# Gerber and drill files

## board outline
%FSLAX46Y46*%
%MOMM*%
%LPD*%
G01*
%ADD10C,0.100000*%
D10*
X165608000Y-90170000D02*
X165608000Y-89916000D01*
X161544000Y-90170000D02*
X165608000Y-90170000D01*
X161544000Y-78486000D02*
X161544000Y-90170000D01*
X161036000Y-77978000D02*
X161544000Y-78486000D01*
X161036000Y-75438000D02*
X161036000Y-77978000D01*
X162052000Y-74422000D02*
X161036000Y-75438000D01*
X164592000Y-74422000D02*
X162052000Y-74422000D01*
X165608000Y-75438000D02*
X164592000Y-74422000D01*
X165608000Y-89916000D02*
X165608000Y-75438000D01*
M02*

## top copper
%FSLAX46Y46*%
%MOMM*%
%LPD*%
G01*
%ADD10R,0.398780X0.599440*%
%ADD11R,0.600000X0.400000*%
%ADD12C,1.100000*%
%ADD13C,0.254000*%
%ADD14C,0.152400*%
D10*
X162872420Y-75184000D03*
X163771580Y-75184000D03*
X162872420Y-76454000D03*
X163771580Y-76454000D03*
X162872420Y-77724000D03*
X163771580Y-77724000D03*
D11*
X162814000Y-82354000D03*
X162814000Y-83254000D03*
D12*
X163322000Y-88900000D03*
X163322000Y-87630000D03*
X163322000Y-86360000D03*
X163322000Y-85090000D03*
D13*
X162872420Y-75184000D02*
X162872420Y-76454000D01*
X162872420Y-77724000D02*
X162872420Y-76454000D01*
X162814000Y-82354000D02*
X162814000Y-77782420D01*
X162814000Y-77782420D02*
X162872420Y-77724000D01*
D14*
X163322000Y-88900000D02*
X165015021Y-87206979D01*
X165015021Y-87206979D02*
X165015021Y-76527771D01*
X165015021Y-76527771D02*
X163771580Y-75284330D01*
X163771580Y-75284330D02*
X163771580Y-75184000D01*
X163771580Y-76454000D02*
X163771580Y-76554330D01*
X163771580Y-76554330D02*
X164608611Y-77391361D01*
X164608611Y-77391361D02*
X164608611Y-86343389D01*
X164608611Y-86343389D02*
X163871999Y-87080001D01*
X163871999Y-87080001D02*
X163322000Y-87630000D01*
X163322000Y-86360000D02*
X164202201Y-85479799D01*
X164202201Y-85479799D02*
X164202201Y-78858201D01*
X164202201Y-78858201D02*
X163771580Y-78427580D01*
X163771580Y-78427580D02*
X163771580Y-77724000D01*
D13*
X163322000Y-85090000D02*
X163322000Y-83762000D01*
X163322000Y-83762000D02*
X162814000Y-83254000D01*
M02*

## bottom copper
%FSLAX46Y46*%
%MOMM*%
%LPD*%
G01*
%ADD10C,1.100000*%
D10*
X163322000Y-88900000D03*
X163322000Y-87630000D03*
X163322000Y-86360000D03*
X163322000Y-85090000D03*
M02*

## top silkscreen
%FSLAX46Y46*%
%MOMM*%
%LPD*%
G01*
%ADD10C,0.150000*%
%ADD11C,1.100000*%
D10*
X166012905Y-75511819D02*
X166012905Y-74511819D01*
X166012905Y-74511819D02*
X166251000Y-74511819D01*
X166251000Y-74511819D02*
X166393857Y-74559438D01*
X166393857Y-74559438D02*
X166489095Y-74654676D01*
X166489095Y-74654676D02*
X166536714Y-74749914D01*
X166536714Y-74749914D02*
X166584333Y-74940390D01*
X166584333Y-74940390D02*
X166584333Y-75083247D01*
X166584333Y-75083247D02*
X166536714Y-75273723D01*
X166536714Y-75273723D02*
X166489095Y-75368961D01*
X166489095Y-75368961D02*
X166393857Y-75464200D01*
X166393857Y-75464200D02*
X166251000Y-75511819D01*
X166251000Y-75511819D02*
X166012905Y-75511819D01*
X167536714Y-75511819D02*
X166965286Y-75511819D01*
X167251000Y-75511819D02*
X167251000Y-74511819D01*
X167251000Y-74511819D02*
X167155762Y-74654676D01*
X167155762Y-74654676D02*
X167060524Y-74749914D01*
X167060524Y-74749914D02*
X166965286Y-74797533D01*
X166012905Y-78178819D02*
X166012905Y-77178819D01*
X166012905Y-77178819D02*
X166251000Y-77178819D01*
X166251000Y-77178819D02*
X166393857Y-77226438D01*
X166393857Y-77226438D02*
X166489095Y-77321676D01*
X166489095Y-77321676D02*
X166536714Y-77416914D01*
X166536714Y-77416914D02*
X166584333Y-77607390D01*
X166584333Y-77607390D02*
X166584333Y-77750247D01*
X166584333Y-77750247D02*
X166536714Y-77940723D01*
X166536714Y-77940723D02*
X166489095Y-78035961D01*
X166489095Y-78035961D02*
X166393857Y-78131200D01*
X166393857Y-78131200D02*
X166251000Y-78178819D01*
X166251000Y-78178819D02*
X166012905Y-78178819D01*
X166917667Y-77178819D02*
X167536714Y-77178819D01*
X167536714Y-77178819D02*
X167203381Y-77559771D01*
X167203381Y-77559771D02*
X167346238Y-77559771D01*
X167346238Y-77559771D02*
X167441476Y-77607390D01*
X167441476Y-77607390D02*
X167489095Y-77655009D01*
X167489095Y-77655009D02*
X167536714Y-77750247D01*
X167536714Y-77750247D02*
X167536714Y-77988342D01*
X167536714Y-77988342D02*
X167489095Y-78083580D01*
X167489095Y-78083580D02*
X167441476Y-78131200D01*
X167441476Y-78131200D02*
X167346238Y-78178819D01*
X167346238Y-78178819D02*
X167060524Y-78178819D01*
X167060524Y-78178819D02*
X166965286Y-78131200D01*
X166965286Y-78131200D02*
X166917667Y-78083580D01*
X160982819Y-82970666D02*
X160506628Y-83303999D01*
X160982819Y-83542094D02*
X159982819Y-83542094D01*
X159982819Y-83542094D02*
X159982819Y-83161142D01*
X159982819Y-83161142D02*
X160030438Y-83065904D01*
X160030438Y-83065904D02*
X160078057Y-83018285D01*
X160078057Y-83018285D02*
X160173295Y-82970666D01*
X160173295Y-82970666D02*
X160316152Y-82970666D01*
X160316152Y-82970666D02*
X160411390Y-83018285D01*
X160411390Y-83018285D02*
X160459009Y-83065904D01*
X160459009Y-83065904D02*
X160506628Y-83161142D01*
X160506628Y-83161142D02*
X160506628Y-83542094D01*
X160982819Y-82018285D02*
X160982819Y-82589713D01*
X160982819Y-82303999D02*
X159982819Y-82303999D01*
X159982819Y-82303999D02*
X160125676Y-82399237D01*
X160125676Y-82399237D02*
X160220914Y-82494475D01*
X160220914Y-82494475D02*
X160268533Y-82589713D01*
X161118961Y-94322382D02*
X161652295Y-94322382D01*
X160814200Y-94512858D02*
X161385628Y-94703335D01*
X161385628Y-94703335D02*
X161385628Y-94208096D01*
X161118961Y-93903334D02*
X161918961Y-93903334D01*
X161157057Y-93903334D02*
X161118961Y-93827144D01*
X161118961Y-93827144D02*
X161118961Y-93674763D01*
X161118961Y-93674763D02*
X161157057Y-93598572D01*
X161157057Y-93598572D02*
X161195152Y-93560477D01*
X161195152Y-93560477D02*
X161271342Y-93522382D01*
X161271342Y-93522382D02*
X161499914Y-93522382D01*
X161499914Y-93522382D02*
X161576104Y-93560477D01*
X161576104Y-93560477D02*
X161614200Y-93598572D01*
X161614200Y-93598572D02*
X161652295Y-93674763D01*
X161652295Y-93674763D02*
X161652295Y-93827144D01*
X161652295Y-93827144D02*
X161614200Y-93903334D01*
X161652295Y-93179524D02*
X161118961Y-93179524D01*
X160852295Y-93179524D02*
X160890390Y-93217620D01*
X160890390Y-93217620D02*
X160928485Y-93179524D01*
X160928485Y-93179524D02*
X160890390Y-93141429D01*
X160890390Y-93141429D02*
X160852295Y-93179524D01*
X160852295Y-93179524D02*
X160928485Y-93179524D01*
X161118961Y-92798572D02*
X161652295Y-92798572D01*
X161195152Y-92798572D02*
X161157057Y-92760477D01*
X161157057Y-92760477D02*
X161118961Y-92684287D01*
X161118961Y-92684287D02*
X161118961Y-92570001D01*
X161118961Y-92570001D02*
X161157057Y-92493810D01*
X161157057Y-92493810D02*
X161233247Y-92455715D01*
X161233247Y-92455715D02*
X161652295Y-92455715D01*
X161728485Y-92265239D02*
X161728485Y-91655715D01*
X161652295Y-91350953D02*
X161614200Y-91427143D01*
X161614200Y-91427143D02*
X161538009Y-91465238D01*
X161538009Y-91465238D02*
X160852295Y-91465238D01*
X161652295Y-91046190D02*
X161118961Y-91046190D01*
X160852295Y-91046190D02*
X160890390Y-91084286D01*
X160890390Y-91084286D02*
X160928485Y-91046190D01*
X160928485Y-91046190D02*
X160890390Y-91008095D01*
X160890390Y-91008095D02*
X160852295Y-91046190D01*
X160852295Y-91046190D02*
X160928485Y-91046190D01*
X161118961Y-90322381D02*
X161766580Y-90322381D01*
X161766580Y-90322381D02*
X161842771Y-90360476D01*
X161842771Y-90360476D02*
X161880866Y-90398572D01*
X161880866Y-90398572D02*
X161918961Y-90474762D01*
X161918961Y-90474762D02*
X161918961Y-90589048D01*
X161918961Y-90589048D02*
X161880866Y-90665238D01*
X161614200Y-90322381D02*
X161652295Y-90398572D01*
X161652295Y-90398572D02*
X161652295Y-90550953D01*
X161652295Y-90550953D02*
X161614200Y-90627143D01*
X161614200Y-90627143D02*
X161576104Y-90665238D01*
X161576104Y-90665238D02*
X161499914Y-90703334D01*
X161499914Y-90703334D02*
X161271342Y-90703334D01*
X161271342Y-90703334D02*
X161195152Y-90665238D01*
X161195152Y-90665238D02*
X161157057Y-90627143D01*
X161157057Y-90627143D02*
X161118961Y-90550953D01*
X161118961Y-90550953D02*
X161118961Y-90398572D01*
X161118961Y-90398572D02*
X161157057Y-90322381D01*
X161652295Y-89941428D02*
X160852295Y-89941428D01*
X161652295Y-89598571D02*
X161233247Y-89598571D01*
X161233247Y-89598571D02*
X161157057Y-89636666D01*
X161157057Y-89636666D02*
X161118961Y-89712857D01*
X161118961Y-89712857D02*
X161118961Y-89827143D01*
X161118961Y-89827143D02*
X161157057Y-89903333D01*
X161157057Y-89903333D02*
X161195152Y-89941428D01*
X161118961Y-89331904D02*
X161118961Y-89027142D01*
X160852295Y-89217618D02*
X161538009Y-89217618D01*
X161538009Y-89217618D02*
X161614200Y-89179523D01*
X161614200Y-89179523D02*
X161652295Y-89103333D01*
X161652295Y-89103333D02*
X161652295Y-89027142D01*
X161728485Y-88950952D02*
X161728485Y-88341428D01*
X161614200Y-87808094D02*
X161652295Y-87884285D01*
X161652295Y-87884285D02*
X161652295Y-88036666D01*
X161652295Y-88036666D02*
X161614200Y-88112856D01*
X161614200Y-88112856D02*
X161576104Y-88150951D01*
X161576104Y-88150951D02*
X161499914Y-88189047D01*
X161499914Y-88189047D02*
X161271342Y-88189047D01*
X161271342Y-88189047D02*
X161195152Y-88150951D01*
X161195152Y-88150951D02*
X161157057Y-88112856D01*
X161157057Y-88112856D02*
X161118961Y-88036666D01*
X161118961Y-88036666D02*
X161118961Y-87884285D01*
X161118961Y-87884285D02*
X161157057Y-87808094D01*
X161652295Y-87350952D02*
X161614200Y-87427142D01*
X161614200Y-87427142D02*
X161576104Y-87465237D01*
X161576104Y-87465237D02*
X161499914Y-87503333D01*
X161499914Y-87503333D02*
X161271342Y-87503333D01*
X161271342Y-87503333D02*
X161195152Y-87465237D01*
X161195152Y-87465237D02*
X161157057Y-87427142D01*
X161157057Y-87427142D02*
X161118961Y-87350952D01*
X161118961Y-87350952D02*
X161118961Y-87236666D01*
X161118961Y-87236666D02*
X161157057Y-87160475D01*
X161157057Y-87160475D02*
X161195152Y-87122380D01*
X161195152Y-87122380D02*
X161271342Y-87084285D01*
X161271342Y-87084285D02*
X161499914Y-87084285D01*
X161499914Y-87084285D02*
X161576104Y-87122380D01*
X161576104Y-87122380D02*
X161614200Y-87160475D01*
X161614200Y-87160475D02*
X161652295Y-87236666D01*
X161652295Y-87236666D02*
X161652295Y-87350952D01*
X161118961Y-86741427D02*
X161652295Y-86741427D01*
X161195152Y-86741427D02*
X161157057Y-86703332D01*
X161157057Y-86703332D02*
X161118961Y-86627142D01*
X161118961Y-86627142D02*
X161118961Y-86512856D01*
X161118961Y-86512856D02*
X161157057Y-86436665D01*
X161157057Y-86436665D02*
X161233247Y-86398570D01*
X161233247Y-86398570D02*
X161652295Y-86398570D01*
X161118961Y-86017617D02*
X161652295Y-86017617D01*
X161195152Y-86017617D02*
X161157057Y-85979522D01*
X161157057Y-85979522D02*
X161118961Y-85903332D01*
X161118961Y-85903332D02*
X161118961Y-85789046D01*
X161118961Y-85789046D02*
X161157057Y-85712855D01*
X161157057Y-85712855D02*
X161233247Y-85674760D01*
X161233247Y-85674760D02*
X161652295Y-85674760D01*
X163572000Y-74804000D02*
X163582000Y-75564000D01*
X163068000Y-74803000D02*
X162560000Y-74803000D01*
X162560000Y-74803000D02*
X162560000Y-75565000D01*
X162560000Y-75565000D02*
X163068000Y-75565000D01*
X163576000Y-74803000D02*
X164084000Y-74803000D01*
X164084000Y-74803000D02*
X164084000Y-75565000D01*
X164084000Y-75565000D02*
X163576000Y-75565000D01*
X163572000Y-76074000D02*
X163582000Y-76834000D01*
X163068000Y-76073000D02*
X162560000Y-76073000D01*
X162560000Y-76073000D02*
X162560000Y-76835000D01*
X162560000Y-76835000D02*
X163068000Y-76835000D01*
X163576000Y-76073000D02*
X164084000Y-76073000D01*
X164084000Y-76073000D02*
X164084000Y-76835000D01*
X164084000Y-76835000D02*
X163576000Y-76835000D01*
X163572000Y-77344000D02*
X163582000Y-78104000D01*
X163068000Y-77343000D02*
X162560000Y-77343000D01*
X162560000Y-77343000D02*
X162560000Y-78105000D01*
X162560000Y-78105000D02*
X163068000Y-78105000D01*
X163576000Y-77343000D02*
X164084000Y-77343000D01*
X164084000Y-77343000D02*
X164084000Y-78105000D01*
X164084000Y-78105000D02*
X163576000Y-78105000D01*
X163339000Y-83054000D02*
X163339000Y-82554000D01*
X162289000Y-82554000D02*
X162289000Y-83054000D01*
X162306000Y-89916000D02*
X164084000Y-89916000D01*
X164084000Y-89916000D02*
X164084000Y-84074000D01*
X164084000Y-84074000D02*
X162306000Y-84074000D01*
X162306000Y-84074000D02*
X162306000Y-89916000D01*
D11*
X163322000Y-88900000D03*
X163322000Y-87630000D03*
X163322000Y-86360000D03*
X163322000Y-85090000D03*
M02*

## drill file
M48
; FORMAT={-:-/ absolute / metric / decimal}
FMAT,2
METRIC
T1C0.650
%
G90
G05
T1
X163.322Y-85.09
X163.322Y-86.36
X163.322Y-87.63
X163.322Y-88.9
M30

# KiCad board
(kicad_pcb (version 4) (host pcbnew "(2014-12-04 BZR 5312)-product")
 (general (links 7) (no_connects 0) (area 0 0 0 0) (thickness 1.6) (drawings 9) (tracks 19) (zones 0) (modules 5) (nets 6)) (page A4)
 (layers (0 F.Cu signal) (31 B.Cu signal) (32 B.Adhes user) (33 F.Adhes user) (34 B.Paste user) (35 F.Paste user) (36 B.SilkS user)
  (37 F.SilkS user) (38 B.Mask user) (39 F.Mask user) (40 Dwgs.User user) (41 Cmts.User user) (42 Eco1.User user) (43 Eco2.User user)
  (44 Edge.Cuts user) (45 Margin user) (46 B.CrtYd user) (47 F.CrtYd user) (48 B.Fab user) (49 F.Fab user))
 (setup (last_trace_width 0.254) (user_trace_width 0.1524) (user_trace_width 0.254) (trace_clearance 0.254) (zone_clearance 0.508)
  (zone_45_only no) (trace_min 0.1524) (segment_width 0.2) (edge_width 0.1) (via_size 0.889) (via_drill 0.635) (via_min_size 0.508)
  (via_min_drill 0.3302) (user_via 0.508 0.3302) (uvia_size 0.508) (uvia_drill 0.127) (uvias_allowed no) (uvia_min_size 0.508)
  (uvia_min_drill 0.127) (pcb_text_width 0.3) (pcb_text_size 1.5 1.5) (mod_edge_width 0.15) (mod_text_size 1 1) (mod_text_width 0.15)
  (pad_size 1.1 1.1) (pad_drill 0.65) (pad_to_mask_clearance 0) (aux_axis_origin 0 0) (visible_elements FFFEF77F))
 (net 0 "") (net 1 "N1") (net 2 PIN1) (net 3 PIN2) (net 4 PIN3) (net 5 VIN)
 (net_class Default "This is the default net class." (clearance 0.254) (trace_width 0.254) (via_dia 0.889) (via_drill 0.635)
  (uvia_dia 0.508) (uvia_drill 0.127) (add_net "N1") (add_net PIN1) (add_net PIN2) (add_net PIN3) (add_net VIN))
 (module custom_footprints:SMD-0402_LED (layer F.Cu) (at 163.322 75.184)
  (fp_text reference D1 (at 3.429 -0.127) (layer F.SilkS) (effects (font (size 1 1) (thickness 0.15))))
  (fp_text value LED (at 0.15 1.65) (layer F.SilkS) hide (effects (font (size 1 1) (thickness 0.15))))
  (fp_line (start 0.25 -0.38) (end 0.26 0.38) (layer F.SilkS) (width 0.15))
  (fp_line (start -0.254 -0.381) (end -0.762 -0.381) (layer F.SilkS) (width 0.15))
  (fp_line (start -0.762 -0.381) (end -0.762 0.381) (layer F.SilkS) (width 0.15))
  (fp_line (start -0.762 0.381) (end -0.254 0.381) (layer F.SilkS) (width 0.15))
  (fp_line (start 0.254 -0.381) (end 0.762 -0.381) (layer F.SilkS) (width 0.15))
  (fp_line (start 0.762 -0.381) (end 0.762 0.381) (layer F.SilkS) (width 0.15))
  (fp_line (start 0.762 0.381) (end 0.254 0.381) (layer F.SilkS) (width 0.15))
  (pad 1 smd rect (at -0.44958 0) (size 0.39878 0.59944) (layers F.Cu F.Paste F.Mask) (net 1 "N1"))
  (pad 2 smd rect (at 0.44958 0) (size 0.39878 0.59944) (layers F.Cu F.Paste F.Mask) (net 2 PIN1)))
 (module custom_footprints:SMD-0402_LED (layer F.Cu) (at 163.322 76.454)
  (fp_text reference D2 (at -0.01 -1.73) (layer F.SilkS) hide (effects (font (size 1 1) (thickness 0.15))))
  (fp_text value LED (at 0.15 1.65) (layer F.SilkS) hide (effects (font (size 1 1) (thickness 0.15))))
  (fp_line (start 0.25 -0.38) (end 0.26 0.38) (layer F.SilkS) (width 0.15))
  (fp_line (start -0.254 -0.381) (end -0.762 -0.381) (layer F.SilkS) (width 0.15))
  (fp_line (start -0.762 -0.381) (end -0.762 0.381) (layer F.SilkS) (width 0.15))
  (fp_line (start -0.762 0.381) (end -0.254 0.381) (layer F.SilkS) (width 0.15))
  (fp_line (start 0.254 -0.381) (end 0.762 -0.381) (layer F.SilkS) (width 0.15))
  (fp_line (start 0.762 -0.381) (end 0.762 0.381) (layer F.SilkS) (width 0.15))
  (fp_line (start 0.762 0.381) (end 0.254 0.381) (layer F.SilkS) (width 0.15))
  (pad 1 smd rect (at -0.44958 0) (size 0.39878 0.59944) (layers F.Cu F.Paste F.Mask) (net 1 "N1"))
  (pad 2 smd rect (at 0.44958 0) (size 0.39878 0.59944) (layers F.Cu F.Paste F.Mask) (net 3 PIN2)))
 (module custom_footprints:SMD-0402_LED (layer F.Cu) (at 163.322 77.724)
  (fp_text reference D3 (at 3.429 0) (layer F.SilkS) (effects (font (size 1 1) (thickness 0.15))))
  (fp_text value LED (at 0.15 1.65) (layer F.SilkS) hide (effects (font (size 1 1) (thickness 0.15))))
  (fp_line (start 0.25 -0.38) (end 0.26 0.38) (layer F.SilkS) (width 0.15))
  (fp_line (start -0.254 -0.381) (end -0.762 -0.381) (layer F.SilkS) (width 0.15))
  (fp_line (start -0.762 -0.381) (end -0.762 0.381) (layer F.SilkS) (width 0.15))
  (fp_line (start -0.762 0.381) (end -0.254 0.381) (layer F.SilkS) (width 0.15))
  (fp_line (start 0.254 -0.381) (end 0.762 -0.381) (layer F.SilkS) (width 0.15))
  (fp_line (start 0.762 -0.381) (end 0.762 0.381) (layer F.SilkS) (width 0.15))
  (fp_line (start 0.762 0.381) (end 0.254 0.381) (layer F.SilkS) (width 0.15))
  (pad 1 smd rect (at -0.44958 0) (size 0.39878 0.59944) (layers F.Cu F.Paste F.Mask) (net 1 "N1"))
  (pad 2 smd rect (at 0.44958 0) (size 0.39878 0.59944) (layers F.Cu F.Paste F.Mask) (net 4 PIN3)))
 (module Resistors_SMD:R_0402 (layer F.Cu) (at 162.814 82.804 270)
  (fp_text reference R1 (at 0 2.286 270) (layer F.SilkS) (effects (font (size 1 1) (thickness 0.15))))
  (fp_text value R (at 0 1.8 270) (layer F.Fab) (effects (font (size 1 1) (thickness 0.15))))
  (fp_line (start 0.25 -0.525) (end -0.25 -0.525) (layer F.SilkS) (width 0.15))
  (fp_line (start -0.25 0.525) (end 0.25 0.525) (layer F.SilkS) (width 0.15))
  (pad 1 smd rect (at -0.45 0 270) (size 0.4 0.6) (layers F.Cu F.Paste F.Mask) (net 1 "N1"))
  (pad 2 smd rect (at 0.45 0 270) (size 0.4 0.6) (layers F.Cu F.Paste F.Mask) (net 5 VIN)))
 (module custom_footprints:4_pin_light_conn (layer F.Cu) (at 167.132 88.9 90)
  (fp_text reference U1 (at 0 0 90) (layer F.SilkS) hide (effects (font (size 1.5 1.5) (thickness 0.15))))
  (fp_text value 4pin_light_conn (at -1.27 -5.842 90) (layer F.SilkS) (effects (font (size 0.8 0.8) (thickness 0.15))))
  (fp_line (start -1.016 -4.826) (end -1.016 -3.048) (layer F.SilkS) (width 0.15))
  (fp_line (start -1.016 -3.048) (end 4.826 -3.048) (layer F.SilkS) (width 0.15))
  (fp_line (start 4.826 -3.048) (end 4.826 -4.826) (layer F.SilkS) (width 0.15))
  (fp_line (start 4.826 -4.826) (end -1.016 -4.826) (layer F.SilkS) (width 0.15))
  (pad 1 thru_hole circle (at 0 -3.81 90) (size 1.1 1.1) (drill 0.65) (layers *.Cu *.Mask F.SilkS) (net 2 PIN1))
  (pad 2 thru_hole circle (at 1.27 -3.81 90) (size 1.1 1.1) (drill 0.65) (layers *.Cu *.Mask F.SilkS) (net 3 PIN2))
  (pad 3 thru_hole circle (at 2.54 -3.81 90) (size 1.1 1.1) (drill 0.65) (layers *.Cu *.Mask F.SilkS) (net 4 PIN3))
  (pad 4 thru_hole circle (at 3.81 -3.81 90) (size 1.1 1.1) (drill 0.65) (layers *.Cu *.Mask F.SilkS) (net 5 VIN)))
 (gr_line (start 165.608 90.17) (end 165.608 89.916) (angle 90) (layer Edge.Cuts) (width 0.1))
 (gr_line (start 161.544 90.17) (end 165.608 90.17) (angle 90) (layer Edge.Cuts) (width 0.1))
 (gr_line (start 161.544 78.486) (end 161.544 90.17) (angle 90) (layer Edge.Cuts) (width 0.1))
 (gr_line (start 161.036 77.978) (end 161.544 78.486) (angle 90) (layer Edge.Cuts) (width 0.1))
 (gr_line (start 161.036 75.438) (end 161.036 77.978) (angle 90) (layer Edge.Cuts) (width 0.1))
 (gr_line (start 162.052 74.422) (end 161.036 75.438) (angle 90) (layer Edge.Cuts) (width 0.1))
 (gr_line (start 164.592 74.422) (end 162.052 74.422) (angle 90) (layer Edge.Cuts) (width 0.1))
 (gr_line (start 165.608 75.438) (end 164.592 74.422) (angle 90) (layer Edge.Cuts) (width 0.1))
 (gr_line (start 165.608 89.916) (end 165.608 75.438) (angle 90) (layer Edge.Cuts) (width 0.1))
 (segment (start 162.87242 75.184) (end 162.87242 76.454) (width 0.254) (layer F.Cu) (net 1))
 (segment (start 162.87242 77.724) (end 162.87242 76.454) (width 0.254) (layer F.Cu) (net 1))
 (segment (start 162.814 82.354) (end 162.814 77.78242) (width 0.254) (layer F.Cu) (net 1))
 (segment (start 162.814 77.78242) (end 162.87242 77.724) (width 0.254) (layer F.Cu) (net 1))
 (segment (start 163.322 88.9) (end 165.015021 87.206979) (width 0.1524) (layer F.Cu) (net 2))
 (segment (start 165.015021 87.206979) (end 165.015021 76.527771) (width 0.1524) (layer F.Cu) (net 2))
 (segment (start 165.015021 76.527771) (end 163.77158 75.28433) (width 0.1524) (layer F.Cu) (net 2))
 (segment (start 163.77158 75.28433) (end 163.77158 75.184) (width 0.1524) (layer F.Cu) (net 2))
 (segment (start 163.77158 76.454) (end 163.77158 76.55433) (width 0.1524) (layer F.Cu) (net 3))
 (segment (start 163.77158 76.55433) (end 164.608611 77.391361) (width 0.1524) (layer F.Cu) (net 3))
 (segment (start 164.608611 77.391361) (end 164.608611 86.343389) (width 0.1524) (layer F.Cu) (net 3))
 (segment (start 164.608611 86.343389) (end 163.871999 87.080001) (width 0.1524) (layer F.Cu) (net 3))
 (segment (start 163.871999 87.080001) (end 163.322 87.63) (width 0.1524) (layer F.Cu) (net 3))
 (segment (start 163.322 86.36) (end 164.202201 85.479799) (width 0.1524) (layer F.Cu) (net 4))
 (segment (start 164.202201 85.479799) (end 164.202201 78.858201) (width 0.1524) (layer F.Cu) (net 4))
 (segment (start 164.202201 78.858201) (end 163.77158 78.42758) (width 0.1524) (layer F.Cu) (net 4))
 (segment (start 163.77158 78.42758) (end 163.77158 77.724) (width 0.1524) (layer F.Cu) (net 4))
 (segment (start 163.322 85.09) (end 163.322 83.762) (width 0.254) (layer F.Cu) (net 5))
 (segment (start 163.322 83.762) (end 162.814 83.254) (width 0.254) (layer F.Cu) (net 5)))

